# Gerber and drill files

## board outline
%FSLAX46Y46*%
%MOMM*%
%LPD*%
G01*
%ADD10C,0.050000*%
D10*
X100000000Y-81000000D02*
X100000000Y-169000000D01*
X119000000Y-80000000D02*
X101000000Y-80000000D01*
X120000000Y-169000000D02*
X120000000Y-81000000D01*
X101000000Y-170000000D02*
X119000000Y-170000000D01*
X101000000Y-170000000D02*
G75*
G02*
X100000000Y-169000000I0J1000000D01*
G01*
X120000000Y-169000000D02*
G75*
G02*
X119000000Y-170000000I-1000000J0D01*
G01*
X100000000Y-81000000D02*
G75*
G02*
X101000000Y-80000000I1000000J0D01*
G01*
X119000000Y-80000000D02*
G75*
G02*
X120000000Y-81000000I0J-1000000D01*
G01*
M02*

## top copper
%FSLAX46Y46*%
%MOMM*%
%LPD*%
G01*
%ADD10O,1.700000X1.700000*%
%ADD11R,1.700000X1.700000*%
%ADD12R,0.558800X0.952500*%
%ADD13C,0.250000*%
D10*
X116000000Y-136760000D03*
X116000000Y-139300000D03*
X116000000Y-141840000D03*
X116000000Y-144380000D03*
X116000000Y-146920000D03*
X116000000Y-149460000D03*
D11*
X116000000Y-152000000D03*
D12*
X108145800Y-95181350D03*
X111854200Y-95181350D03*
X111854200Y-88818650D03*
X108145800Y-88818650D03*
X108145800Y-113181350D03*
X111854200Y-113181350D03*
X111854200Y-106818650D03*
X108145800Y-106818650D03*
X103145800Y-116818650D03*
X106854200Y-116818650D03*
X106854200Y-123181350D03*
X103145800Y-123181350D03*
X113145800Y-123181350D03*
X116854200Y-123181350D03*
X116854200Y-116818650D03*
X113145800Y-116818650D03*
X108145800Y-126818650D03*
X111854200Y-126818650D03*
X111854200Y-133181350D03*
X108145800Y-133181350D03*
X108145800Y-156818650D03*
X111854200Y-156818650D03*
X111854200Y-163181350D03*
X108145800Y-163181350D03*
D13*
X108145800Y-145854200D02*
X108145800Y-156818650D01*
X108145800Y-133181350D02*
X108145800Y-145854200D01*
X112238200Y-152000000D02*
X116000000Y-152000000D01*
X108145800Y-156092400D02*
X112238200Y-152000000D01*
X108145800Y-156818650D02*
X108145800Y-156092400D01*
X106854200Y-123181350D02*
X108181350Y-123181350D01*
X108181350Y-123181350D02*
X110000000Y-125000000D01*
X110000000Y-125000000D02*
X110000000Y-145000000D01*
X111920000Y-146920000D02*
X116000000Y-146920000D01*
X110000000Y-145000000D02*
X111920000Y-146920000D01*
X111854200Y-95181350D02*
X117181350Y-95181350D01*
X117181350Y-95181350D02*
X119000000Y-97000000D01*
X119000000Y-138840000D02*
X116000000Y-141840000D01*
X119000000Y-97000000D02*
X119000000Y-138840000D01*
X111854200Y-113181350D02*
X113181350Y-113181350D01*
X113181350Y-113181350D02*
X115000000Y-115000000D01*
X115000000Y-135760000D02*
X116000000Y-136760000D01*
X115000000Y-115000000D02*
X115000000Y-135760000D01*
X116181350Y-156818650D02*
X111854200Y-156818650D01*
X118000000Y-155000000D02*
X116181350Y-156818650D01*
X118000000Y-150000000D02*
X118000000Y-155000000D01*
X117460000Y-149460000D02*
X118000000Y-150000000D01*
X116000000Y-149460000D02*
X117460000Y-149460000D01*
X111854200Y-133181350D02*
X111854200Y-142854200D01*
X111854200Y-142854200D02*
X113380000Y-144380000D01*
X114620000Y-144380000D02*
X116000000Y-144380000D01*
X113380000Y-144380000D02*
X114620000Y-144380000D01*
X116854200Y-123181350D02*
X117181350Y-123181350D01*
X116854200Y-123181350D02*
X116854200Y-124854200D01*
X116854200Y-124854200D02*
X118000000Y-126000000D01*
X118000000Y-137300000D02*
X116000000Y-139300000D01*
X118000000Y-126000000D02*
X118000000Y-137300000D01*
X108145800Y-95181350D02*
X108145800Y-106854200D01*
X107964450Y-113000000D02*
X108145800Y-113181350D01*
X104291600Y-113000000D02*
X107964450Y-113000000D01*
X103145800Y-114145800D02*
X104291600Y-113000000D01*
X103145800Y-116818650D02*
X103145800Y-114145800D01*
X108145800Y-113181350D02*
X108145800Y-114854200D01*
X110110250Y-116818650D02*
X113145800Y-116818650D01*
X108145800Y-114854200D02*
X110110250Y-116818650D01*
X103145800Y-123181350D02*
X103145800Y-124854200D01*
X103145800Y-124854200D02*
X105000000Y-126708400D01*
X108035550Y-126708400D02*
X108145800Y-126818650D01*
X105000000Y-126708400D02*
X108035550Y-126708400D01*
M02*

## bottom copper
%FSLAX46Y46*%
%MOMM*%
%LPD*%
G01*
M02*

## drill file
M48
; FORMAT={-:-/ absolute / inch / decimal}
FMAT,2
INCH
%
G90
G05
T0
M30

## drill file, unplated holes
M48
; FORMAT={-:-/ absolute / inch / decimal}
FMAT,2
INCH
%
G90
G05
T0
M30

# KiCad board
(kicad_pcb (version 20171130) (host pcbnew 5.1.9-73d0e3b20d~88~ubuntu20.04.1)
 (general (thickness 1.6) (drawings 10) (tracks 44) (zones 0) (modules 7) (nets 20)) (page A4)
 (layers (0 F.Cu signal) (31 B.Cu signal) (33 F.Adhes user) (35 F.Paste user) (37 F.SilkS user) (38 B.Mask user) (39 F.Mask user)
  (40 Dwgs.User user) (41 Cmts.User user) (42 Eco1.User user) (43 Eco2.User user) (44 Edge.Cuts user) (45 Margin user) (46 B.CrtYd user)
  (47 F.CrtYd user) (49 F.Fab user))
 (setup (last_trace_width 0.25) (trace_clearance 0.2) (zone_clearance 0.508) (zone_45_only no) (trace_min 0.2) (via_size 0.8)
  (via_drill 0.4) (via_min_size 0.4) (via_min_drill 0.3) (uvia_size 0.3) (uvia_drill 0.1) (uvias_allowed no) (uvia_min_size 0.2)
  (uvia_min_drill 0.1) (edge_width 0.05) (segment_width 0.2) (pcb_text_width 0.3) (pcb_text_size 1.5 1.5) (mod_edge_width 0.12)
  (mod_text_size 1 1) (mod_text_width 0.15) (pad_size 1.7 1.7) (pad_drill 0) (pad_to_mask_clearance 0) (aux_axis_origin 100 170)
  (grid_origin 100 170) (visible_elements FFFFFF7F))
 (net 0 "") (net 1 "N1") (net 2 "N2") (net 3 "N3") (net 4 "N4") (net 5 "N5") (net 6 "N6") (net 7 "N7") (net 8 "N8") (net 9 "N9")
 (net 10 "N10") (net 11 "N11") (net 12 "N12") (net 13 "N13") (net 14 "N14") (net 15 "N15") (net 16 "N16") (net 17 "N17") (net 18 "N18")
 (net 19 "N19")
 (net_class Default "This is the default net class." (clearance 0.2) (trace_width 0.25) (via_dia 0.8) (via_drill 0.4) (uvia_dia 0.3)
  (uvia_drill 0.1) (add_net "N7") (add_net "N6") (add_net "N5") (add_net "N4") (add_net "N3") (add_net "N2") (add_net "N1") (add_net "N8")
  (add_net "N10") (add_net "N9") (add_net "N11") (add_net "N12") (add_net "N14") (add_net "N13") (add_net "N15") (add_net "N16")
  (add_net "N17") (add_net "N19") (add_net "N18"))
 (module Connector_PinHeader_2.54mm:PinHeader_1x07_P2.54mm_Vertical (layer F.Cu) (at 116 152 180)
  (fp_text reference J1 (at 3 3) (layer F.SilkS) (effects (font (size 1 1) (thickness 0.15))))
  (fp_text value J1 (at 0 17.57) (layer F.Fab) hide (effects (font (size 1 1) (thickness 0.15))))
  (pad 7 smd oval (at 0 15.24 180) (size 1.7 1.7) (layers F.Cu F.Paste F.Mask) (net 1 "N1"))
  (pad 6 smd oval (at 0 12.7 180) (size 1.7 1.7) (layers F.Cu F.Paste F.Mask) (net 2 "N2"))
  (pad 5 smd oval (at 0 10.16 180) (size 1.7 1.7) (layers F.Cu F.Paste F.Mask) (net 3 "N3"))
  (pad 4 smd oval (at 0 7.62 180) (size 1.7 1.7) (layers F.Cu F.Paste F.Mask) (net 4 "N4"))
  (pad 3 smd oval (at 0 5.08 180) (size 1.7 1.7) (layers F.Cu F.Paste F.Mask) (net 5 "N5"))
  (pad 2 smd oval (at 0 2.54 180) (size 1.7 1.7) (layers F.Cu F.Paste F.Mask) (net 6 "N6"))
  (pad 1 smd rect (at 0 0 180) (size 1.7 1.7) (layers F.Cu F.Paste F.Mask) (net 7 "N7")))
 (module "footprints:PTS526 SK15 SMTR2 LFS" (layer F.Cu) (at 110 92 90)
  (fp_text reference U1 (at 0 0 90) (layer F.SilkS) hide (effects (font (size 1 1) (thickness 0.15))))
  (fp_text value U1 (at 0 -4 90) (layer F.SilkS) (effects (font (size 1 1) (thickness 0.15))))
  (pad 1 smd rect (at -3.18135 -1.8542 90) (size 0.9525 0.5588) (layers F.Cu F.Paste F.Mask) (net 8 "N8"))
  (pad 3 smd rect (at -3.18135 1.8542 90) (size 0.9525 0.5588) (layers F.Cu F.Paste F.Mask) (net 3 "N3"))
  (pad 4 smd rect (at 3.18135 1.8542 90) (size 0.9525 0.5588) (layers F.Cu F.Paste F.Mask) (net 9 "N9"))
  (pad 2 smd rect (at 3.18135 -1.8542 90) (size 0.9525 0.5588) (layers F.Cu F.Paste F.Mask) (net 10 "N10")))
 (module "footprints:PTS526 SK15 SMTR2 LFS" (layer F.Cu) (at 110 110 90)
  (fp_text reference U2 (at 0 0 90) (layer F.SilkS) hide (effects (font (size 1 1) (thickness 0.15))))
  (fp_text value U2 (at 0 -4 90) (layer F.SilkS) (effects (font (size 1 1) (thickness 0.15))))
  (pad 1 smd rect (at -3.18135 -1.8542 90) (size 0.9525 0.5588) (layers F.Cu F.Paste F.Mask) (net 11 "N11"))
  (pad 3 smd rect (at -3.18135 1.8542 90) (size 0.9525 0.5588) (layers F.Cu F.Paste F.Mask) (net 1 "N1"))
  (pad 4 smd rect (at 3.18135 1.8542 90) (size 0.9525 0.5588) (layers F.Cu F.Paste F.Mask) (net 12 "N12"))
  (pad 2 smd rect (at 3.18135 -1.8542 90) (size 0.9525 0.5588) (layers F.Cu F.Paste F.Mask) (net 8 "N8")))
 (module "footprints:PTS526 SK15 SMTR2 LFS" (layer F.Cu) (at 105 120 90)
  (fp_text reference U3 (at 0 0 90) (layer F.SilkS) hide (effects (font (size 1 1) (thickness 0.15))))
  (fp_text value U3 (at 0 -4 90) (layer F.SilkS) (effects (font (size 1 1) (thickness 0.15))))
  (pad 2 smd rect (at 3.18135 -1.8542 90) (size 0.9525 0.5588) (layers F.Cu F.Paste F.Mask) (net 11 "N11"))
  (pad 4 smd rect (at 3.18135 1.8542 90) (size 0.9525 0.5588) (layers F.Cu F.Paste F.Mask) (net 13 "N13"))
  (pad 3 smd rect (at -3.18135 1.8542 90) (size 0.9525 0.5588) (layers F.Cu F.Paste F.Mask) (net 5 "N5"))
  (pad 1 smd rect (at -3.18135 -1.8542 90) (size 0.9525 0.5588) (layers F.Cu F.Paste F.Mask) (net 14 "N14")))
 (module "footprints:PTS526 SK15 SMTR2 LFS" (layer F.Cu) (at 115 120 90)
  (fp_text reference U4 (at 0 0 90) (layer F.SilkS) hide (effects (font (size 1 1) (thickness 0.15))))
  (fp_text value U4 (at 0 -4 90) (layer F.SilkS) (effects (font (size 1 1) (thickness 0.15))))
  (pad 1 smd rect (at -3.18135 -1.8542 90) (size 0.9525 0.5588) (layers F.Cu F.Paste F.Mask) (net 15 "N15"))
  (pad 3 smd rect (at -3.18135 1.8542 90) (size 0.9525 0.5588) (layers F.Cu F.Paste F.Mask) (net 2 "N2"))
  (pad 4 smd rect (at 3.18135 1.8542 90) (size 0.9525 0.5588) (layers F.Cu F.Paste F.Mask) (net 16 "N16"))
  (pad 2 smd rect (at 3.18135 -1.8542 90) (size 0.9525 0.5588) (layers F.Cu F.Paste F.Mask) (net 11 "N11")))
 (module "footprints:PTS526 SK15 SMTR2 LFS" (layer F.Cu) (at 110 130 90)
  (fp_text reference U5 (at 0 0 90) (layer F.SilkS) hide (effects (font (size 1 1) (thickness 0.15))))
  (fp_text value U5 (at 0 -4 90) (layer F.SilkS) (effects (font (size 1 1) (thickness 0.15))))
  (pad 2 smd rect (at 3.18135 -1.8542 90) (size 0.9525 0.5588) (layers F.Cu F.Paste F.Mask) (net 14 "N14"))
  (pad 4 smd rect (at 3.18135 1.8542 90) (size 0.9525 0.5588) (layers F.Cu F.Paste F.Mask) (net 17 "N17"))
  (pad 3 smd rect (at -3.18135 1.8542 90) (size 0.9525 0.5588) (layers F.Cu F.Paste F.Mask) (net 4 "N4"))
  (pad 1 smd rect (at -3.18135 -1.8542 90) (size 0.9525 0.5588) (layers F.Cu F.Paste F.Mask) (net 7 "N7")))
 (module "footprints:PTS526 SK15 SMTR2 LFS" (layer F.Cu) (at 110 160 90)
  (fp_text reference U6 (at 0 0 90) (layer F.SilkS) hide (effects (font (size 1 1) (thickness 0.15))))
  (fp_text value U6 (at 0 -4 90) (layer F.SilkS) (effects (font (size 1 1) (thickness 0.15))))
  (pad 2 smd rect (at 3.18135 -1.8542 90) (size 0.9525 0.5588) (layers F.Cu F.Paste F.Mask) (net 7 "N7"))
  (pad 4 smd rect (at 3.18135 1.8542 90) (size 0.9525 0.5588) (layers F.Cu F.Paste F.Mask) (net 6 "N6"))
  (pad 3 smd rect (at -3.18135 1.8542 90) (size 0.9525 0.5588) (layers F.Cu F.Paste F.Mask) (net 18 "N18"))
  (pad 1 smd rect (at -3.18135 -1.8542 90) (size 0.9525 0.5588) (layers F.Cu F.Paste F.Mask) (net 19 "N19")))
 (gr_line (start 100 81) (end 100 169) (layer Edge.Cuts) (width 0.05))
 (gr_line (start 119 80) (end 101 80) (layer Edge.Cuts) (width 0.05))
 (gr_line (start 120 169) (end 120 81) (layer Edge.Cuts) (width 0.05))
 (gr_line (start 101 170) (end 119 170) (layer Edge.Cuts) (width 0.05))
 (gr_arc (start 101 169) (end 100 169) (angle -90) (layer Edge.Cuts) (width 0.05))
 (gr_arc (start 119 169) (end 119 170) (angle -90) (layer Edge.Cuts) (width 0.05))
 (gr_arc (start 101 81) (end 101 80) (angle -90) (layer Edge.Cuts) (width 0.05))
 (gr_arc (start 119 81) (end 120 81) (angle -90) (layer Edge.Cuts) (width 0.05))
 (segment (start 108.1458 145.8542) (end 108.1458 156.81865) (width 0.25) (layer F.Cu) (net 7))
 (segment (start 108.1458 133.18135) (end 108.1458 145.8542) (width 0.25) (layer F.Cu) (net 7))
 (segment (start 112.2382 152) (end 116 152) (width 0.25) (layer F.Cu) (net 7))
 (segment (start 108.1458 156.0924) (end 112.2382 152) (width 0.25) (layer F.Cu) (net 7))
 (segment (start 108.1458 156.81865) (end 108.1458 156.0924) (width 0.25) (layer F.Cu) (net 7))
 (segment (start 106.8542 123.18135) (end 108.18135 123.18135) (width 0.25) (layer F.Cu) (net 5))
 (segment (start 108.18135 123.18135) (end 110 125) (width 0.25) (layer F.Cu) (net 5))
 (segment (start 110 125) (end 110 145) (width 0.25) (layer F.Cu) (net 5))
 (segment (start 111.92 146.92) (end 116 146.92) (width 0.25) (layer F.Cu) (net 5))
 (segment (start 110 145) (end 111.92 146.92) (width 0.25) (layer F.Cu) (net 5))
 (segment (start 111.8542 95.18135) (end 117.18135 95.18135) (width 0.25) (layer F.Cu) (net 3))
 (segment (start 117.18135 95.18135) (end 119 97) (width 0.25) (layer F.Cu) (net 3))
 (segment (start 119 138.84) (end 116 141.84) (width 0.25) (layer F.Cu) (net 3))
 (segment (start 119 97) (end 119 138.84) (width 0.25) (layer F.Cu) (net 3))
 (segment (start 111.8542 113.18135) (end 113.18135 113.18135) (width 0.25) (layer F.Cu) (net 1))
 (segment (start 113.18135 113.18135) (end 115 115) (width 0.25) (layer F.Cu) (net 1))
 (segment (start 115 135.76) (end 116 136.76) (width 0.25) (layer F.Cu) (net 1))
 (segment (start 115 115) (end 115 135.76) (width 0.25) (layer F.Cu) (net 1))
 (segment (start 116.18135 156.81865) (end 111.8542 156.81865) (width 0.25) (layer F.Cu) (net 6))
 (segment (start 118 155) (end 116.18135 156.81865) (width 0.25) (layer F.Cu) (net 6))
 (segment (start 118 150) (end 118 155) (width 0.25) (layer F.Cu) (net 6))
 (segment (start 117.46 149.46) (end 118 150) (width 0.25) (layer F.Cu) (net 6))
 (segment (start 116 149.46) (end 117.46 149.46) (width 0.25) (layer F.Cu) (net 6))
 (segment (start 111.8542 133.18135) (end 111.8542 142.8542) (width 0.25) (layer F.Cu) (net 4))
 (segment (start 111.8542 142.8542) (end 113.38 144.38) (width 0.25) (layer F.Cu) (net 4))
 (segment (start 114.62 144.38) (end 116 144.38) (width 0.25) (layer F.Cu) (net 4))
 (segment (start 113.38 144.38) (end 114.62 144.38) (width 0.25) (layer F.Cu) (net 4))
 (segment (start 116.8542 123.18135) (end 117.18135 123.18135) (width 0.25) (layer F.Cu) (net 2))
 (segment (start 116.8542 123.18135) (end 116.8542 124.8542) (width 0.25) (layer F.Cu) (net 2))
 (segment (start 116.8542 124.8542) (end 118 126) (width 0.25) (layer F.Cu) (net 2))
 (segment (start 118 137.3) (end 116 139.3) (width 0.25) (layer F.Cu) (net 2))
 (segment (start 118 126) (end 118 137.3) (width 0.25) (layer F.Cu) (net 2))
 (segment (start 108.1458 95.18135) (end 108.1458 106.8542) (width 0.25) (layer F.Cu) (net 8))
 (segment (start 107.96445 113) (end 108.1458 113.18135) (width 0.25) (layer F.Cu) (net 11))
 (segment (start 104.2916 113) (end 107.96445 113) (width 0.25) (layer F.Cu) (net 11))
 (segment (start 103.1458 114.1458) (end 104.2916 113) (width 0.25) (layer F.Cu) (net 11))
 (segment (start 103.1458 116.81865) (end 103.1458 114.1458) (width 0.25) (layer F.Cu) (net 11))
 (segment (start 108.1458 113.18135) (end 108.1458 114.8542) (width 0.25) (layer F.Cu) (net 11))
 (segment (start 110.11025 116.81865) (end 113.1458 116.81865) (width 0.25) (layer F.Cu) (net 11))
 (segment (start 108.1458 114.8542) (end 110.11025 116.81865) (width 0.25) (layer F.Cu) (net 11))
 (segment (start 103.1458 123.18135) (end 103.1458 124.8542) (width 0.25) (layer F.Cu) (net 14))
 (segment (start 103.1458 124.8542) (end 105 126.7084) (width 0.25) (layer F.Cu) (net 14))
 (segment (start 108.03555 126.7084) (end 108.1458 126.81865) (width 0.25) (layer F.Cu) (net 14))
 (segment (start 105 126.7084) (end 108.03555 126.7084) (width 0.25) (layer F.Cu) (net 14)))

